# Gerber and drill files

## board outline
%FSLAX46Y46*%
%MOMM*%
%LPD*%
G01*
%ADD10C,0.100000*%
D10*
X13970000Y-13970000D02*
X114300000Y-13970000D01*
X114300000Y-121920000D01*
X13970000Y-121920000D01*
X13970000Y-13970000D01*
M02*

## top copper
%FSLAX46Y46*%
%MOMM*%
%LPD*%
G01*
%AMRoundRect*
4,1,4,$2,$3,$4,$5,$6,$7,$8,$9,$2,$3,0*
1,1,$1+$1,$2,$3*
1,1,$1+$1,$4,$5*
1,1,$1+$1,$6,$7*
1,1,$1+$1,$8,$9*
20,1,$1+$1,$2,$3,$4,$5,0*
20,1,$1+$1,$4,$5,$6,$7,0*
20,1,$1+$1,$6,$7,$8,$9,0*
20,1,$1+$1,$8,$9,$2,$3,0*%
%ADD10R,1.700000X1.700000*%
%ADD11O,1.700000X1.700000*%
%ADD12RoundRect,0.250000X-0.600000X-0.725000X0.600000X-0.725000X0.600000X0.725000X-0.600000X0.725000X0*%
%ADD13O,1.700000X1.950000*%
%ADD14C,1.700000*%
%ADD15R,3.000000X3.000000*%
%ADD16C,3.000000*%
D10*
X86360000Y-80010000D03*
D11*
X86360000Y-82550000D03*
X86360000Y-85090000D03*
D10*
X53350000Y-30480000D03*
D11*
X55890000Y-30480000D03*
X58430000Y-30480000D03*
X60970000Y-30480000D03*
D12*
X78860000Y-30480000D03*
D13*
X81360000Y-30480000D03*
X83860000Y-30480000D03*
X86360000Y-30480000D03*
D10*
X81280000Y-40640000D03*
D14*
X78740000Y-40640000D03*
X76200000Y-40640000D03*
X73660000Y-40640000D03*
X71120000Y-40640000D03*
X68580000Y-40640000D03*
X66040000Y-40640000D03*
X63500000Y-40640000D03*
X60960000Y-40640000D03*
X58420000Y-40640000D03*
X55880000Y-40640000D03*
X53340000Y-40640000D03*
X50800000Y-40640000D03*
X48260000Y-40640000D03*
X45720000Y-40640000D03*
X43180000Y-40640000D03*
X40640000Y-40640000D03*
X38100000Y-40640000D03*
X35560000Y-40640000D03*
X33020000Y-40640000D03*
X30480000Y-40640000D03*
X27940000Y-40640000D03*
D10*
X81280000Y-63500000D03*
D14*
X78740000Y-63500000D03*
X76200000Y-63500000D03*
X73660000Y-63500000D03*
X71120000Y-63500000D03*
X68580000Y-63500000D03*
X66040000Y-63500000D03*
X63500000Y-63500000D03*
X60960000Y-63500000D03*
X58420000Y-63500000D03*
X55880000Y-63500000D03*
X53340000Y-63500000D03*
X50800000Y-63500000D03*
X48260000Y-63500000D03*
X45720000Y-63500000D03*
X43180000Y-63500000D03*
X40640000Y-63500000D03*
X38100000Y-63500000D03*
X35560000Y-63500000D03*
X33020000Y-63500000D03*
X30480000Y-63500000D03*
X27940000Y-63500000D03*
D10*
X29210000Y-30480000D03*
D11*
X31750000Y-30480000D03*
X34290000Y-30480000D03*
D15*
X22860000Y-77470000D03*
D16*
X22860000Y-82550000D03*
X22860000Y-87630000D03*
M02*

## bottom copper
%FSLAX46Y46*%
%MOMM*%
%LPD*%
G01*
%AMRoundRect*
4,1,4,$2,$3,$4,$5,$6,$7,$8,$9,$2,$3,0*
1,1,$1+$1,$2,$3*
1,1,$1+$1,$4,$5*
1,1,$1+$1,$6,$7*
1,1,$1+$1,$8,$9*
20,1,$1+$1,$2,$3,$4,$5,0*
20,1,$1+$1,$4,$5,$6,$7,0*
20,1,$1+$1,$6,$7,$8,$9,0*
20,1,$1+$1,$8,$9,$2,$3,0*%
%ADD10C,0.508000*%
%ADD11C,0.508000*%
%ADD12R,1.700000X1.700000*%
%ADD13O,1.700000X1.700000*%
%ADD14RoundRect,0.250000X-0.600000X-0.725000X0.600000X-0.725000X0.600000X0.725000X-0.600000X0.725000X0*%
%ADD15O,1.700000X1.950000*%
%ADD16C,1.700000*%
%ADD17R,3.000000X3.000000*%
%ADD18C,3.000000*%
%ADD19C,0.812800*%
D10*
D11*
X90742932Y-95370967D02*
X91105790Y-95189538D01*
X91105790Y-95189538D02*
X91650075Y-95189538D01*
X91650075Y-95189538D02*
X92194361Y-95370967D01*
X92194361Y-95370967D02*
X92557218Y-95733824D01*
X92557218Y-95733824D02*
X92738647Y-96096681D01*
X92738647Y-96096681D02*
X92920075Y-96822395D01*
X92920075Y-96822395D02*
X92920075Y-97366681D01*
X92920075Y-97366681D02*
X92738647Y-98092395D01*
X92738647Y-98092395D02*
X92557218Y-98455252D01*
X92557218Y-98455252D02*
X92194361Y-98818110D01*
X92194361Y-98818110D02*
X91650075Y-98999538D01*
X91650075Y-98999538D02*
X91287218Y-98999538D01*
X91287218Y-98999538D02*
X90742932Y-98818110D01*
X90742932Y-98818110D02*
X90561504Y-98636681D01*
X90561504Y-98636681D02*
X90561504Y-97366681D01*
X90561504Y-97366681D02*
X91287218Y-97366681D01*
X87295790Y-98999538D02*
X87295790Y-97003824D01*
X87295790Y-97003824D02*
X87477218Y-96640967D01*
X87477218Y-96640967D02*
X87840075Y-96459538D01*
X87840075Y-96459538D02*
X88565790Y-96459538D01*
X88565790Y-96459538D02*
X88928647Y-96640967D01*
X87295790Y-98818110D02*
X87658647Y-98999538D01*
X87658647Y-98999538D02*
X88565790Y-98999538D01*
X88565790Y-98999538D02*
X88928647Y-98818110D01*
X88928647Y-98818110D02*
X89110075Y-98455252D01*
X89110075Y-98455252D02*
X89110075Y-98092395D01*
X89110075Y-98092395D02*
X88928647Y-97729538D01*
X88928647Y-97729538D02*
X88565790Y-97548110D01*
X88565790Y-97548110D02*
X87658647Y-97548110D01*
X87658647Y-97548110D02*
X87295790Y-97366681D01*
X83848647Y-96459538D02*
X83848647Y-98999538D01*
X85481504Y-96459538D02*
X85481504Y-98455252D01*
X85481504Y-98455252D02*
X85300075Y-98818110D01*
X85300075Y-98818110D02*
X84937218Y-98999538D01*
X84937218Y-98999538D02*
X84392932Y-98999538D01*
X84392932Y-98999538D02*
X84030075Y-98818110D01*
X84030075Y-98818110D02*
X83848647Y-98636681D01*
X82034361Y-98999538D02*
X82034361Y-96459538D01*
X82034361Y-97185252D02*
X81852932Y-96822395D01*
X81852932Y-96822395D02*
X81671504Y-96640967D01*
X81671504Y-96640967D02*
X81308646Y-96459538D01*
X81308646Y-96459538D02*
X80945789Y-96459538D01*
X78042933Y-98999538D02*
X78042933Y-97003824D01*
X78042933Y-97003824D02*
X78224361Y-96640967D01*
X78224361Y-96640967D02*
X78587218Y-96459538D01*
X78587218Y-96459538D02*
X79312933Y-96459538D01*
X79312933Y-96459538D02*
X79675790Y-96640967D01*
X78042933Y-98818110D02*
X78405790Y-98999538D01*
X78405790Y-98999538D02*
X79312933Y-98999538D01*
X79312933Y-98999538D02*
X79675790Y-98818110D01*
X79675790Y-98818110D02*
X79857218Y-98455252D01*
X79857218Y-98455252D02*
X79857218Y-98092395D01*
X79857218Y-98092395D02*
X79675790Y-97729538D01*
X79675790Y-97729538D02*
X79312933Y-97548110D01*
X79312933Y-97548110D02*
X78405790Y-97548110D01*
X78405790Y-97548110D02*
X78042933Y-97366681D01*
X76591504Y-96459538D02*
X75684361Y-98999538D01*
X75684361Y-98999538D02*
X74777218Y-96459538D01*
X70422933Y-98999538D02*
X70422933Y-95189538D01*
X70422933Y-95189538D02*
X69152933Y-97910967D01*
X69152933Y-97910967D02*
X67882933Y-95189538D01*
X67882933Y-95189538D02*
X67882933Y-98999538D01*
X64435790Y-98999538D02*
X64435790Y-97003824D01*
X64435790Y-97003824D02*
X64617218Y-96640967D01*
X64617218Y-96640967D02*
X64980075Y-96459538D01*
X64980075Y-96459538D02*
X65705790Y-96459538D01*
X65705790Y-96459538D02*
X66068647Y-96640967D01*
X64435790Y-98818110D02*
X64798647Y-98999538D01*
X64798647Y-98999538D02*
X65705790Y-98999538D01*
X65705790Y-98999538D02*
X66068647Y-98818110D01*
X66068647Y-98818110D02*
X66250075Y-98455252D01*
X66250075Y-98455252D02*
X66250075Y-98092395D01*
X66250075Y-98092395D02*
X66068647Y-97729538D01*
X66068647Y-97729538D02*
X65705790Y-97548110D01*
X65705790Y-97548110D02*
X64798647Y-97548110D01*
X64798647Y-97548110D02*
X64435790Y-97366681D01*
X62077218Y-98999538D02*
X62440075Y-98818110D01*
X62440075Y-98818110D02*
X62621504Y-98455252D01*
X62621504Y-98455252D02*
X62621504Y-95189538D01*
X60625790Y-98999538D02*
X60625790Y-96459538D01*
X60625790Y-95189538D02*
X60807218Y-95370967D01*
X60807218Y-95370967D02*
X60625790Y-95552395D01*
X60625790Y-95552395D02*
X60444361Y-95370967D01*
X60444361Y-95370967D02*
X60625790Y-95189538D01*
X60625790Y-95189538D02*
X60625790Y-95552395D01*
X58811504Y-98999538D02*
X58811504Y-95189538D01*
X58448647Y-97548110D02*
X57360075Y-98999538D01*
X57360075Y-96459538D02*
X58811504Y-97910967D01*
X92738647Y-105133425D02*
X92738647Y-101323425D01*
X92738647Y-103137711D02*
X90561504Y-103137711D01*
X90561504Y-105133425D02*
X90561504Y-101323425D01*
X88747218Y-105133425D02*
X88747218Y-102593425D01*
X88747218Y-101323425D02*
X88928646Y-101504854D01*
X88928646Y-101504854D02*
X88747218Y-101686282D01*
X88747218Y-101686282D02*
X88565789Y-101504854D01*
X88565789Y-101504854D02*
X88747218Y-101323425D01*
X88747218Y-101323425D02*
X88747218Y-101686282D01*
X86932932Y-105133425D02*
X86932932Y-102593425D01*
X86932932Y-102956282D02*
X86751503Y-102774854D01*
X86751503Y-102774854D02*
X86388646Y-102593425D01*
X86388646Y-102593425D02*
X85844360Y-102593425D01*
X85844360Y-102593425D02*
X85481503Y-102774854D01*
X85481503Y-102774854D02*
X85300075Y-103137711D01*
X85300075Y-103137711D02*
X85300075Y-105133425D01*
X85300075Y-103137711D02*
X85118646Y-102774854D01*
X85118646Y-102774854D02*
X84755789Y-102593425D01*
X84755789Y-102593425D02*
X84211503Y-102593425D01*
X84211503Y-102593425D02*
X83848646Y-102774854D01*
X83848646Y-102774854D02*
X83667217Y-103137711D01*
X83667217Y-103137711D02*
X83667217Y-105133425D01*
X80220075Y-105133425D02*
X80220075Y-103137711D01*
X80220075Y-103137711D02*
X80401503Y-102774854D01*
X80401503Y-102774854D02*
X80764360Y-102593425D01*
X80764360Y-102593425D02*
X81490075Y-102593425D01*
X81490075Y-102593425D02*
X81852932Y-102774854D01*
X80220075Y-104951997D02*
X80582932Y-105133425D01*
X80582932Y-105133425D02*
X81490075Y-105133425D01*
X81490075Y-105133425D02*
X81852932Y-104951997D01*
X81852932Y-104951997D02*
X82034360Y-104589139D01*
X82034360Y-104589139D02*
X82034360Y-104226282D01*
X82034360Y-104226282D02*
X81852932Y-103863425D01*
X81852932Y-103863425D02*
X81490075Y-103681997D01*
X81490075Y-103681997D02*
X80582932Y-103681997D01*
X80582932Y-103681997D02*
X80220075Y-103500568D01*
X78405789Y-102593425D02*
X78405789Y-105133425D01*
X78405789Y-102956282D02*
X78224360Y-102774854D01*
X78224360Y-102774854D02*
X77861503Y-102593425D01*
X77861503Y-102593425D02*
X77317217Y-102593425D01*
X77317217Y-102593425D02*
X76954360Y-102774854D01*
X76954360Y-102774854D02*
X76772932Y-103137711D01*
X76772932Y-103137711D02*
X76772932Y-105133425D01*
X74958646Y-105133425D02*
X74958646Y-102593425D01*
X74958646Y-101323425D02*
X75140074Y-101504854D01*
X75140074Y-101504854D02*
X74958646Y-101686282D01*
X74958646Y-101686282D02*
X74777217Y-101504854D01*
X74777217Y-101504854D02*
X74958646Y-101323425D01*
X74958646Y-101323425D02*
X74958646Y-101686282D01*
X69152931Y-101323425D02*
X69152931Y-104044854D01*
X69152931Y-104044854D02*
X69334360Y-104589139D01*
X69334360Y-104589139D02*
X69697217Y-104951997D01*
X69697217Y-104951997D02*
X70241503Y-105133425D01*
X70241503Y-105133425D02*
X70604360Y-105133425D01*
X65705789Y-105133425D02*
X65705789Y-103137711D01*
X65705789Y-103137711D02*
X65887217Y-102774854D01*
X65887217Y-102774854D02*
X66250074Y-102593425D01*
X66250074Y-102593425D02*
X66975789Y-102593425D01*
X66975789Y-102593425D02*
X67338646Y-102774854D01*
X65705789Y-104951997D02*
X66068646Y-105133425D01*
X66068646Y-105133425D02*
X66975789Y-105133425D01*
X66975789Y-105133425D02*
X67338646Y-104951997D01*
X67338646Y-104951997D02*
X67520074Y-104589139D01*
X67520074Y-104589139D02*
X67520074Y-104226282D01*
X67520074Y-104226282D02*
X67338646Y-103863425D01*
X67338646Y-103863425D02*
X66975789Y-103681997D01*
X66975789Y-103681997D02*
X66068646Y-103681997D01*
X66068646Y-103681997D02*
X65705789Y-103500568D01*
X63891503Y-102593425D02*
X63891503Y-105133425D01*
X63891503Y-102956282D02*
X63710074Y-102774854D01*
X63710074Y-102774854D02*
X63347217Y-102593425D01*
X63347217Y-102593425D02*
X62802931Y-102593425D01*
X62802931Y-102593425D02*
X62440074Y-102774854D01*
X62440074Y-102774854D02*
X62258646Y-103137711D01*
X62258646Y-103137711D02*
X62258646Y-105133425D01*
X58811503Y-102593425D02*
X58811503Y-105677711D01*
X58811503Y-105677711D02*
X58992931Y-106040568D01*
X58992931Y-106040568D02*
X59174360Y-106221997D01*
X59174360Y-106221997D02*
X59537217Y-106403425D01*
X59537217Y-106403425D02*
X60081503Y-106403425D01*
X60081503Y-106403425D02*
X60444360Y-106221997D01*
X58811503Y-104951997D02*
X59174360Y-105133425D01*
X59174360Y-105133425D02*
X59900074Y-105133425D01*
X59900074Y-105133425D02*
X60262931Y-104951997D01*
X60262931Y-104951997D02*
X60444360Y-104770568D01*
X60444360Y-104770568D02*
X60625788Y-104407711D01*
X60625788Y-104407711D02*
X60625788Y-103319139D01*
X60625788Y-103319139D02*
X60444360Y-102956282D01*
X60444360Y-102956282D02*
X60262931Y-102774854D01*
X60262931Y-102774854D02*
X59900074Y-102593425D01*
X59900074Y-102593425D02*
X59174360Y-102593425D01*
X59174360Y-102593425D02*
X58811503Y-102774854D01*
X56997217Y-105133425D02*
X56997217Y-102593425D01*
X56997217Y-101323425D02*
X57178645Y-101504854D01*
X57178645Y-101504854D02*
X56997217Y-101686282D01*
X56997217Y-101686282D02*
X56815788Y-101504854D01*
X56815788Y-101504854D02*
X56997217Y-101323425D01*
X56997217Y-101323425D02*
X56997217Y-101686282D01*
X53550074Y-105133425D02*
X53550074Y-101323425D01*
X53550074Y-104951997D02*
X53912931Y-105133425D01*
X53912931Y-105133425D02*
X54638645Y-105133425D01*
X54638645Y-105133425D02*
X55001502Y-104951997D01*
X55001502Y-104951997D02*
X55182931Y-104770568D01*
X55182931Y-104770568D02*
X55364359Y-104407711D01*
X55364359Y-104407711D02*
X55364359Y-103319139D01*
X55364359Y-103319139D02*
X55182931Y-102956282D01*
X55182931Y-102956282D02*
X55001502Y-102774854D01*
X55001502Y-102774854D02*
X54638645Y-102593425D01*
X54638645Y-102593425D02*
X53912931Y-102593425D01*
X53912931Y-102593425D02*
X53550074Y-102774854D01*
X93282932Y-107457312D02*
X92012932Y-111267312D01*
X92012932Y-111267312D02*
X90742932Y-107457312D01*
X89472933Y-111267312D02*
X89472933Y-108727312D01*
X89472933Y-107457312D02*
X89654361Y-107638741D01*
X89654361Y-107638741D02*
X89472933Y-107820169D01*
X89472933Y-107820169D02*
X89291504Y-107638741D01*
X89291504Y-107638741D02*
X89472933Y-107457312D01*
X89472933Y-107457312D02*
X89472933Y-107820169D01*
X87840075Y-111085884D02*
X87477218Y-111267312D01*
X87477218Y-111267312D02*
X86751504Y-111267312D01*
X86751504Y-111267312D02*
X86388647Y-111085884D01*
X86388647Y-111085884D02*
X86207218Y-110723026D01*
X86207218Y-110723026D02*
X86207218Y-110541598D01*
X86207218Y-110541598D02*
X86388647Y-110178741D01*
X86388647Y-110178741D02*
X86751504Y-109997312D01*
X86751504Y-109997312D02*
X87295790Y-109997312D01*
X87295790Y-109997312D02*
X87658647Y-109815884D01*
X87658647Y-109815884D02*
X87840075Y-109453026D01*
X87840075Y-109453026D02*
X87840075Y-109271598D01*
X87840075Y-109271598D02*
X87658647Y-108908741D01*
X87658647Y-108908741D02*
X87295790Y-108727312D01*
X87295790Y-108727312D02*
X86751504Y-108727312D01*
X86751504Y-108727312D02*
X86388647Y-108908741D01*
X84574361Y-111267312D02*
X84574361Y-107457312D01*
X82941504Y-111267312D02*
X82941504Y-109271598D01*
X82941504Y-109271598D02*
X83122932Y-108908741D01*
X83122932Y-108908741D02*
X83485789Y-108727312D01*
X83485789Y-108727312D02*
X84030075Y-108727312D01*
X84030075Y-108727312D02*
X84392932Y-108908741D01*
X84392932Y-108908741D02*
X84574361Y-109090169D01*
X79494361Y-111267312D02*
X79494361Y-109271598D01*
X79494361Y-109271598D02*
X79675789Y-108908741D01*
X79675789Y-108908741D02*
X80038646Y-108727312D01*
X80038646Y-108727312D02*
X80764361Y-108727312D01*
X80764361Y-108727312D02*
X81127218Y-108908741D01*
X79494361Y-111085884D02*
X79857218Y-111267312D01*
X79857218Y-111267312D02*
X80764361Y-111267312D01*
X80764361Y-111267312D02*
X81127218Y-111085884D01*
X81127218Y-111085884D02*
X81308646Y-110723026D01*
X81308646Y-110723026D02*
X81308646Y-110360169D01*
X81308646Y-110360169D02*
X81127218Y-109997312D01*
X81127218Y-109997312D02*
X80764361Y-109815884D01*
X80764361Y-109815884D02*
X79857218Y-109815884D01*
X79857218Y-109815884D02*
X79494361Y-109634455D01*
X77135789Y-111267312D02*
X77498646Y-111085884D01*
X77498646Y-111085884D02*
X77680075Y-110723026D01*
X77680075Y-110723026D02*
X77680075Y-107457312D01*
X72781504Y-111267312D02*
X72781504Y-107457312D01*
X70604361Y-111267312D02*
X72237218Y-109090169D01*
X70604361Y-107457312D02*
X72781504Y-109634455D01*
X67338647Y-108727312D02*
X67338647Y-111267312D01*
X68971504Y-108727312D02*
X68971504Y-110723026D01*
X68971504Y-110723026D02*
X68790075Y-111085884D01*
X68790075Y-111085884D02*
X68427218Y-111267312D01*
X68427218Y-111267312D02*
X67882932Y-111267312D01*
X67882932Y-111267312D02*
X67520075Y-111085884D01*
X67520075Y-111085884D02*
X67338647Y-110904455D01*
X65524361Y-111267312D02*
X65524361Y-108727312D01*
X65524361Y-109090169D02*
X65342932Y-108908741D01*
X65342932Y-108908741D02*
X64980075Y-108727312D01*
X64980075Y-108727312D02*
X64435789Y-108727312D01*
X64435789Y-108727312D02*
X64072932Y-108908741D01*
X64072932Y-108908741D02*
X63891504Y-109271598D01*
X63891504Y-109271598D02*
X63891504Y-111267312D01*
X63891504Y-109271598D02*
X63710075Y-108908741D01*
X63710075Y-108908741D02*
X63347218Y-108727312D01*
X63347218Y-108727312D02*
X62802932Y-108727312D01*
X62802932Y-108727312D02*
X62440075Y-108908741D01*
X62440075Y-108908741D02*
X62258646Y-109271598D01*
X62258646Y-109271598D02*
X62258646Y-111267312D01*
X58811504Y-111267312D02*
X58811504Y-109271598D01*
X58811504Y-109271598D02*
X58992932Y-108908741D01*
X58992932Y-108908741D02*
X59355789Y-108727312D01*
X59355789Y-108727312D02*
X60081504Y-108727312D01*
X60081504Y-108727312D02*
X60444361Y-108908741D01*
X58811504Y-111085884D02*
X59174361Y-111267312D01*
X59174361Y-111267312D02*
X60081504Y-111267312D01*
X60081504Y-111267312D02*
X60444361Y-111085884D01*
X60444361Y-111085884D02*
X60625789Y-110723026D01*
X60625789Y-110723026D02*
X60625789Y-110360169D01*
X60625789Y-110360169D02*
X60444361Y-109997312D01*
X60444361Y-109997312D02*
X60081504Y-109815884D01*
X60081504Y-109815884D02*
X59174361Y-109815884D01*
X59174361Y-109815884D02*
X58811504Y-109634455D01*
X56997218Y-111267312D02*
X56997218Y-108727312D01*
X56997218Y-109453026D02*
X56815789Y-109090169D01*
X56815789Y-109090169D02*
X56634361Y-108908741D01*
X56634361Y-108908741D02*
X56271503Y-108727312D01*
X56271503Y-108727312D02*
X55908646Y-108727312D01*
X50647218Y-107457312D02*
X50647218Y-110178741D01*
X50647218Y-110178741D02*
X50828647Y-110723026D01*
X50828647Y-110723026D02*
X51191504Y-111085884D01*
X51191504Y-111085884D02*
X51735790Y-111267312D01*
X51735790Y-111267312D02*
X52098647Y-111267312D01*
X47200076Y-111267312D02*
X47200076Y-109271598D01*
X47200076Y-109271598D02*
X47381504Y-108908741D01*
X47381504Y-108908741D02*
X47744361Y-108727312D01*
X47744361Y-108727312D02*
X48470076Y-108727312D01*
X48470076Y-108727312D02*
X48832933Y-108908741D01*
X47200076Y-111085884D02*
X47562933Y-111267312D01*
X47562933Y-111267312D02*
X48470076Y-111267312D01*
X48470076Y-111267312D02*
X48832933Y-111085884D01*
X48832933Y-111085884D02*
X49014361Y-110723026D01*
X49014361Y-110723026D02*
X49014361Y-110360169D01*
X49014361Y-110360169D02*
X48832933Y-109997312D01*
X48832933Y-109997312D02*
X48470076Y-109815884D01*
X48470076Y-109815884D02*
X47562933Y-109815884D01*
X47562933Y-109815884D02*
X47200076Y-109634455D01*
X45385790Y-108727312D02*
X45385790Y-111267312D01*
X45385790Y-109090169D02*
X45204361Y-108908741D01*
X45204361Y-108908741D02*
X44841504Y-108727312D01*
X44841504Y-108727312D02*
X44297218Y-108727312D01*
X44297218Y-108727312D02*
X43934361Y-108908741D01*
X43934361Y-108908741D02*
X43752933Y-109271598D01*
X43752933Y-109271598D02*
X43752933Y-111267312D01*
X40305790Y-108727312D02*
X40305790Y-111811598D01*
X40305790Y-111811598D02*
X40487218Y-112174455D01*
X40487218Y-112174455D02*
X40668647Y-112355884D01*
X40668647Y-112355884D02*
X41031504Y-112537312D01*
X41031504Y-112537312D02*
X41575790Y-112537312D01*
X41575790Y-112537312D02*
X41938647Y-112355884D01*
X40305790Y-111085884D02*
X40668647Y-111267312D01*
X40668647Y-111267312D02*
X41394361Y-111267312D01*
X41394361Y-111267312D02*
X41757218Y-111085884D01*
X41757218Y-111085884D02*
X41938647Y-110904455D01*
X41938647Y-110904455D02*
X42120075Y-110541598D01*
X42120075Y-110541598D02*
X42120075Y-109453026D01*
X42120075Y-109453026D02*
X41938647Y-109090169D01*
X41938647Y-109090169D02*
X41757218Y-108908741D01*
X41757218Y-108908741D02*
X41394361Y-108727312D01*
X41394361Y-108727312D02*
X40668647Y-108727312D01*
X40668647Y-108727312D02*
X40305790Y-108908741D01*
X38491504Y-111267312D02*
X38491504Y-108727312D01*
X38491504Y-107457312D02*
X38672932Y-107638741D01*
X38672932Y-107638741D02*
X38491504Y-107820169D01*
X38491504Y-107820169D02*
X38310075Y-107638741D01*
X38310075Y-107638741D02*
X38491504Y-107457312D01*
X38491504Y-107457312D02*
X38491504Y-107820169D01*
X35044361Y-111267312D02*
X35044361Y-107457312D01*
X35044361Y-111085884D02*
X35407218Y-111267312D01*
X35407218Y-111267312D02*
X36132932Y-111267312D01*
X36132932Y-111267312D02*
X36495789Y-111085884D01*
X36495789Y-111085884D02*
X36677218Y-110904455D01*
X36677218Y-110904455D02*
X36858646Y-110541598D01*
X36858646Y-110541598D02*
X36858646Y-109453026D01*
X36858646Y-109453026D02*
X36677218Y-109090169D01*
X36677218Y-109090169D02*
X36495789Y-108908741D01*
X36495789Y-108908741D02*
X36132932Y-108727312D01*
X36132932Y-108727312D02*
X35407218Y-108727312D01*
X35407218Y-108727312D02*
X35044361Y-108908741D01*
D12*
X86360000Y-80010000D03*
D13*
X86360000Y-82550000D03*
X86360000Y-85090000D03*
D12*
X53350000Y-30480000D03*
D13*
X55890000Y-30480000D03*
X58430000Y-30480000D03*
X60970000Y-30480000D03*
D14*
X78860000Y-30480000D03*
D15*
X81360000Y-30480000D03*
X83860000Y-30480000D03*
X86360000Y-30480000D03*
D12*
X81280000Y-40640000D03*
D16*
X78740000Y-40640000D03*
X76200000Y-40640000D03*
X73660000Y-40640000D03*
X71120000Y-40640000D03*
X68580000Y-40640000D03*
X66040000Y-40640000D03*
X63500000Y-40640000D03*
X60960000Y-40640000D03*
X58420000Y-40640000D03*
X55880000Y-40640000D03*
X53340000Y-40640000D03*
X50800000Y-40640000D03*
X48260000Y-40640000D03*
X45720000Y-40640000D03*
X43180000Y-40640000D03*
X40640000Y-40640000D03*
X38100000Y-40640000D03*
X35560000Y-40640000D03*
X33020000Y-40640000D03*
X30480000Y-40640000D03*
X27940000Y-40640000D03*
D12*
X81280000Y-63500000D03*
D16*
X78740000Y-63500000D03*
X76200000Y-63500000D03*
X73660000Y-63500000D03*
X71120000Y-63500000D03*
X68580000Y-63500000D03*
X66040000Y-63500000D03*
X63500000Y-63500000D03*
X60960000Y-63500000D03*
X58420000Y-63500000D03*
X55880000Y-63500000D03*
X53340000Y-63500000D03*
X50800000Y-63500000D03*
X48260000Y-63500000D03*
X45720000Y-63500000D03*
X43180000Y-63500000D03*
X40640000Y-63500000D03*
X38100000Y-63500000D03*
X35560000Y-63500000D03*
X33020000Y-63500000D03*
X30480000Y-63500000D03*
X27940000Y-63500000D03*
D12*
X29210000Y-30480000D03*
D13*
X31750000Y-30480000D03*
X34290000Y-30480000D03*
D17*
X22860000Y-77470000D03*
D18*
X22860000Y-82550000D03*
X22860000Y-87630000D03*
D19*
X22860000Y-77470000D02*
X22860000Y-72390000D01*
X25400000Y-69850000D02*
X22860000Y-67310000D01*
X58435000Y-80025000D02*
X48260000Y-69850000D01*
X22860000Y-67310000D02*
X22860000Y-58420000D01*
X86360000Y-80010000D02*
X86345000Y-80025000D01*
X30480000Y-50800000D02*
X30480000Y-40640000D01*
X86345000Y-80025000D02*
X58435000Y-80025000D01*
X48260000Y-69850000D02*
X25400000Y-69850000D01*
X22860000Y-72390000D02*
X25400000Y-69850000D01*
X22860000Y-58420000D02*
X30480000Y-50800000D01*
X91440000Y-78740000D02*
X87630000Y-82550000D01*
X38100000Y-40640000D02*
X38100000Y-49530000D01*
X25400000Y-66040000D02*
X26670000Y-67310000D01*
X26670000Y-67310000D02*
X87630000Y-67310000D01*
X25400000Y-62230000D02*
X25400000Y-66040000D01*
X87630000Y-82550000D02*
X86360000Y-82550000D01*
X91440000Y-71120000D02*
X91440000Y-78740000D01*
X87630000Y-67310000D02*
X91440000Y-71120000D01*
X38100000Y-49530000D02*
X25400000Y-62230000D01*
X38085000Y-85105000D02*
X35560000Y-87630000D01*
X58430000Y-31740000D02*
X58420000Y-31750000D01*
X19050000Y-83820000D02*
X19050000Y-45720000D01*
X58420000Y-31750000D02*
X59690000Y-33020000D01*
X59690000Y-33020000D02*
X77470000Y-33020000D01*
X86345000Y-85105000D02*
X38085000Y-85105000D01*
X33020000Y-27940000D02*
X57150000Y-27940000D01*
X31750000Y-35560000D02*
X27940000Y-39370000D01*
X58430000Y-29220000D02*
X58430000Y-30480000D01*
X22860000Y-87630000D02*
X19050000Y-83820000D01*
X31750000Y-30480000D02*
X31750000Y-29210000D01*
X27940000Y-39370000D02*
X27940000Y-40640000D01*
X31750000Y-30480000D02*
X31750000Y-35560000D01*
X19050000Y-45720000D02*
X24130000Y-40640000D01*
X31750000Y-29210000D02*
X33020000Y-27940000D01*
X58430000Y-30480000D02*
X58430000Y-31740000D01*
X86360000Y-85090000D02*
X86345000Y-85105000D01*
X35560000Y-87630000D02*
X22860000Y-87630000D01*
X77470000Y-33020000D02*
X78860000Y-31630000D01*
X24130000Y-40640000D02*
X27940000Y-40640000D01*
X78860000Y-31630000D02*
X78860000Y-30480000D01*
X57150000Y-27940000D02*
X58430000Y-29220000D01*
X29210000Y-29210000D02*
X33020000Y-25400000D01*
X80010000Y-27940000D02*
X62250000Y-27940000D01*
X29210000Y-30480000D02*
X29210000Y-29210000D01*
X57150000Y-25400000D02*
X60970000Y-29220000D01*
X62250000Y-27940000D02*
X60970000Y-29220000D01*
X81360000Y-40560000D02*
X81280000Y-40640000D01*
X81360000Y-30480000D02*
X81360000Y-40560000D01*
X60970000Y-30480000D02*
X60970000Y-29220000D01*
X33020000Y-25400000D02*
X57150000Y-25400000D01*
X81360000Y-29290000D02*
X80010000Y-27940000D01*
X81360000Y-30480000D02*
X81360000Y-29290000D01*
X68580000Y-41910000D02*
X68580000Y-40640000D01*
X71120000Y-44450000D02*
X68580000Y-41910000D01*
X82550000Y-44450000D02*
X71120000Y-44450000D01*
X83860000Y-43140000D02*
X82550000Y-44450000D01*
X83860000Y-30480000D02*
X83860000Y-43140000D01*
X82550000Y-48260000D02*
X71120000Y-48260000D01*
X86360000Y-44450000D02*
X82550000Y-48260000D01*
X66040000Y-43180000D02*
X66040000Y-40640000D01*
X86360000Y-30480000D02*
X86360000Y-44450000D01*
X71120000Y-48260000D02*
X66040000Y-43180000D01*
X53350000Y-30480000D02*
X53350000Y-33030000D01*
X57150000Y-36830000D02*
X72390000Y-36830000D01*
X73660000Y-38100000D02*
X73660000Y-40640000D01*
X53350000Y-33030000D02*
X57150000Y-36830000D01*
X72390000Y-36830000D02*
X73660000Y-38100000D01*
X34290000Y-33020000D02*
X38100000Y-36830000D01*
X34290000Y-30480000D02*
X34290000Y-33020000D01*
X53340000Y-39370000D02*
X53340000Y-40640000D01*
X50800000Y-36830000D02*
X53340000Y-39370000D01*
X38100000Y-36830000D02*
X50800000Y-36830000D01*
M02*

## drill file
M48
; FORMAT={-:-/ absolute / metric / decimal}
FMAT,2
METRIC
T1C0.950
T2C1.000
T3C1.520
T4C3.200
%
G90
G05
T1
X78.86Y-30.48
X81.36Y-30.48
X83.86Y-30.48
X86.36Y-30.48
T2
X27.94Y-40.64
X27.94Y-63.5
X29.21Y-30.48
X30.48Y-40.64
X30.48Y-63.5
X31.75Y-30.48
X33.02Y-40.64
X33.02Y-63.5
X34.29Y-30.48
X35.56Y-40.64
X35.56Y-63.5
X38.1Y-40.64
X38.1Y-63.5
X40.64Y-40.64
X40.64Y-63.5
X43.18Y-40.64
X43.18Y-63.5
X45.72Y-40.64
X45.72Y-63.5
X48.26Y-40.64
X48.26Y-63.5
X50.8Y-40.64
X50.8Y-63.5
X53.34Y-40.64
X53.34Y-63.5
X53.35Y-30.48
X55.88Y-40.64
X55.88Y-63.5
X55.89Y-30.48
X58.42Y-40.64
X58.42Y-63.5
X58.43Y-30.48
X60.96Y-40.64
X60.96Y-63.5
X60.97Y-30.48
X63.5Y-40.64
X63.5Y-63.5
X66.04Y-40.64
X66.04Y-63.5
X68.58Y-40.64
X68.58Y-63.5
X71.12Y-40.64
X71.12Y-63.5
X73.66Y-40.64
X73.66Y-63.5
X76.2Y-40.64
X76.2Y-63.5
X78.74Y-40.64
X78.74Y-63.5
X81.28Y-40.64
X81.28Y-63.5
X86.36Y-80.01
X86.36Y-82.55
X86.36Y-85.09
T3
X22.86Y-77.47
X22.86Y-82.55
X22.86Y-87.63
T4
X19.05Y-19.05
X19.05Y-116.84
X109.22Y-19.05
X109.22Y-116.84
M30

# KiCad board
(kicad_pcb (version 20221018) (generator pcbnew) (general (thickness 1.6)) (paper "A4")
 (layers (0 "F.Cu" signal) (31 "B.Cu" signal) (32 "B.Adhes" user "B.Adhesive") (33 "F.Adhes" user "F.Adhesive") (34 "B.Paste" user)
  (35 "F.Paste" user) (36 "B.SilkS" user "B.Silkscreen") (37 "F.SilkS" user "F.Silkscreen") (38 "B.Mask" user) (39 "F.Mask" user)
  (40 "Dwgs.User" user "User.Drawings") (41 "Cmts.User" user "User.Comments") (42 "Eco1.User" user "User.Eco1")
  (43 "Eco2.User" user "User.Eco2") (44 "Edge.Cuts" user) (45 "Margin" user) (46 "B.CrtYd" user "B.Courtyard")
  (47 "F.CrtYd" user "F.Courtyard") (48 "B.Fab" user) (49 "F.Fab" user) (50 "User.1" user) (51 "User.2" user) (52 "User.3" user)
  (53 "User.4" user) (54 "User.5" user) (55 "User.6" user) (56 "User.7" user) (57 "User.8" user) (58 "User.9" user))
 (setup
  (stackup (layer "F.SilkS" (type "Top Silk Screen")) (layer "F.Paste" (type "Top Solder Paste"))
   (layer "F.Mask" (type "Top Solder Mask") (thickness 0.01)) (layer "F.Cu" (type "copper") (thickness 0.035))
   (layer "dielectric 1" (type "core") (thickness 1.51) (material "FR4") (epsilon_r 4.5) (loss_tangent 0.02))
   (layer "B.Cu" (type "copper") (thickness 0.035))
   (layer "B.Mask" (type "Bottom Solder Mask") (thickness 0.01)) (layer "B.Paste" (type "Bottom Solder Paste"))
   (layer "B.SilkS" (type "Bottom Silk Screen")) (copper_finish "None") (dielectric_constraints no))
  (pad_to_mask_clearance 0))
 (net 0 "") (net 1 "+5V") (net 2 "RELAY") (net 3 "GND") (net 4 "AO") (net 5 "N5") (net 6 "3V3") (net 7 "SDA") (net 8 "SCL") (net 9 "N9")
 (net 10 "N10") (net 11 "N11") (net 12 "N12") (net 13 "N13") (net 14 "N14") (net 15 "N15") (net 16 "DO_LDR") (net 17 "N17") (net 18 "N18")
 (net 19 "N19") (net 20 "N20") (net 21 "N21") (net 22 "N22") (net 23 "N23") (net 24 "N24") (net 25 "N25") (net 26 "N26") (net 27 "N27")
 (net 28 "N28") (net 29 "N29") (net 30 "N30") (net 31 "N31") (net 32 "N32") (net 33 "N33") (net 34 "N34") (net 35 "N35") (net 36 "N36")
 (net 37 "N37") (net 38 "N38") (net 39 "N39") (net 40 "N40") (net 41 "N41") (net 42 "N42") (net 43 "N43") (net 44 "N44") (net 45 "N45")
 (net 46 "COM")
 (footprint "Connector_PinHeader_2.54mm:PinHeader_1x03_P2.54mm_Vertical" (layer "F.Cu") (at 86.36 80.01)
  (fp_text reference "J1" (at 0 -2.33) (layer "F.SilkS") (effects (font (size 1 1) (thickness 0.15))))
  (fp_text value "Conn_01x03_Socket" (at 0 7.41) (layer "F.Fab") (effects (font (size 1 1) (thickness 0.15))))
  (pad "1" thru_hole rect (at 0 0) (size 1.7 1.7) (drill 1) (layers "*.Cu" "*.Mask") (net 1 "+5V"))
  (pad "2" thru_hole oval (at 0 2.54) (size 1.7 1.7) (drill 1) (layers "*.Cu" "*.Mask") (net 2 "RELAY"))
  (pad "3" thru_hole oval (at 0 5.08) (size 1.7 1.7) (drill 1) (layers "*.Cu" "*.Mask") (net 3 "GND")))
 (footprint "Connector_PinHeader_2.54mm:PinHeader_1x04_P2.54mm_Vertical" (layer "F.Cu") (at 53.35 30.48 90)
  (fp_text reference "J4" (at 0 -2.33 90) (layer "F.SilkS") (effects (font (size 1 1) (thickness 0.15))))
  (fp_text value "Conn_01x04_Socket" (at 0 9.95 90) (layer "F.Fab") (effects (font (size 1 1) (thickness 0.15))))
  (pad "1" thru_hole rect (at 0 0 90) (size 1.7 1.7) (drill 1) (layers "*.Cu" "*.Mask") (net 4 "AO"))
  (pad "2" thru_hole oval (at 0 2.54 90) (size 1.7 1.7) (drill 1) (layers "*.Cu" "*.Mask") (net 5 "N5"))
  (pad "3" thru_hole oval (at 0 5.08 90) (size 1.7 1.7) (drill 1) (layers "*.Cu" "*.Mask") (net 3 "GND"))
  (pad "4" thru_hole oval (at 0 7.62 90) (size 1.7 1.7) (drill 1) (layers "*.Cu" "*.Mask") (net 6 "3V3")))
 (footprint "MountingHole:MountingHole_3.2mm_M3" (layer "F.Cu") (at 109.22 19.05)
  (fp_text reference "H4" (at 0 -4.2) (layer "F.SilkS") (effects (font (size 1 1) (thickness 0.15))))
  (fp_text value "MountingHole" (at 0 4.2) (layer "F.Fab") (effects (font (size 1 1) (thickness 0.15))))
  (pad "" np_thru_hole circle (at 0 0) (size 3.2 3.2) (drill 3.2) (layers "*.Cu" "*.Mask")))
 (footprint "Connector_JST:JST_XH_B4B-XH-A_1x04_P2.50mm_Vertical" (layer "F.Cu") (at 78.86 30.48)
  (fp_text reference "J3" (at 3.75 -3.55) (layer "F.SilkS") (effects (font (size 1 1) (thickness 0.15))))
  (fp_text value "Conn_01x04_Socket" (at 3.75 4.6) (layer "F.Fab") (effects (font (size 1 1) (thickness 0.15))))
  (pad "1" thru_hole roundrect (at 0 0) (size 1.7 1.95) (drill 0.95) (layers "*.Cu" "*.Mask") (roundrect_rratio 0.147059) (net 3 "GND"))
  (pad "2" thru_hole oval (at 2.5 0) (size 1.7 1.95) (drill 0.95) (layers "*.Cu" "*.Mask") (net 6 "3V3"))
  (pad "3" thru_hole oval (at 5 0) (size 1.7 1.95) (drill 0.95) (layers "*.Cu" "*.Mask") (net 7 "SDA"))
  (pad "4" thru_hole oval (at 7.5 0) (size 1.7 1.95) (drill 0.95) (layers "*.Cu" "*.Mask") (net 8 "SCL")))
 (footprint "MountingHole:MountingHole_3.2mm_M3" (layer "F.Cu") (at 19.05 19.05)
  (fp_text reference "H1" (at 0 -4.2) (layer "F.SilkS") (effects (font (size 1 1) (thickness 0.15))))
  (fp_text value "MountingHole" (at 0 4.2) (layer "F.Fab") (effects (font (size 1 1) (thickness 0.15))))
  (pad "" np_thru_hole circle (at 0 0) (size 3.2 3.2) (drill 3.2) (layers "*.Cu" "*.Mask")))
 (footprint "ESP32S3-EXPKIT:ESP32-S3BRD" (layer "F.Cu") (at 16.48 39.37 -90)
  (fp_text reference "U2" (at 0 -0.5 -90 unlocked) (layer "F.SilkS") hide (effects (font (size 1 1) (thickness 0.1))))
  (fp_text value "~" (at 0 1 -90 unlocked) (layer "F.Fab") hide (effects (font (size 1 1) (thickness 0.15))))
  (pad "1_1" thru_hole rect (at 1.27 -64.8 270) (size 1.7 1.7) (drill 1) (layers "*.Cu" "*.Mask") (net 6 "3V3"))
  (pad "1_2" thru_hole circle (at 1.27 -62.26 270) (size 1.7 1.7) (drill 1) (layers "*.Cu" "*.Mask") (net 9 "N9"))
  (pad "1_3" thru_hole circle (at 1.27 -59.72 270) (size 1.7 1.7) (drill 1) (layers "*.Cu" "*.Mask") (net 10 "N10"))
  (pad "1_4" thru_hole circle (at 1.27 -57.18 270) (size 1.7 1.7) (drill 1) (layers "*.Cu" "*.Mask") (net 4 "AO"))
  (pad "1_5" thru_hole circle (at 1.27 -54.64 270) (size 1.7 1.7) (drill 1) (layers "*.Cu" "*.Mask") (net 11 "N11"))
  (pad "1_6" thru_hole circle (at 1.27 -52.1 270) (size 1.7 1.7) (drill 1) (layers "*.Cu" "*.Mask") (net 7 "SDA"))
  (pad "1_7" thru_hole circle (at 1.27 -49.56 270) (size 1.7 1.7) (drill 1) (layers "*.Cu" "*.Mask") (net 8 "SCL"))
  (pad "1_8" thru_hole circle (at 1.27 -47.02 270) (size 1.7 1.7) (drill 1) (layers "*.Cu" "*.Mask") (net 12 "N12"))
  (pad "1_9" thru_hole circle (at 1.27 -44.48 270) (size 1.7 1.7) (drill 1) (layers "*.Cu" "*.Mask") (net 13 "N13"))
  (pad "1_10" thru_hole circle (at 1.27 -41.94 270) (size 1.7 1.7) (drill 1) (layers "*.Cu" "*.Mask") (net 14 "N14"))
  (pad "1_11" thru_hole circle (at 1.27 -39.4 270) (size 1.7 1.7) (drill 1) (layers "*.Cu" "*.Mask") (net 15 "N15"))
  (pad "1_12" thru_hole circle (at 1.27 -36.86 270) (size 1.7 1.7) (drill 1) (layers "*.Cu" "*.Mask") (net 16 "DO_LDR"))
  (pad "1_13" thru_hole circle (at 1.27 -34.32 270) (size 1.7 1.7) (drill 1) (layers "*.Cu" "*.Mask") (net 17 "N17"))
  (pad "1_14" thru_hole circle (at 1.27 -31.78 270) (size 1.7 1.7) (drill 1) (layers "*.Cu" "*.Mask") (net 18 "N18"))
  (pad "1_15" thru_hole circle (at 1.27 -29.24 270) (size 1.7 1.7) (drill 1) (layers "*.Cu" "*.Mask") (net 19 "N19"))
  (pad "1_16" thru_hole circle (at 1.27 -26.7 270) (size 1.7 1.7) (drill 1) (layers "*.Cu" "*.Mask") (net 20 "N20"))
  (pad "1_17" thru_hole circle (at 1.27 -24.16 270) (size 1.7 1.7) (drill 1) (layers "*.Cu" "*.Mask") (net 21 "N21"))
  (pad "1_18" thru_hole circle (at 1.27 -21.62 270) (size 1.7 1.7) (drill 1) (layers "*.Cu" "*.Mask") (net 2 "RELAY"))
  (pad "1_19" thru_hole circle (at 1.27 -19.08 270) (size 1.7 1.7) (drill 1) (layers "*.Cu" "*.Mask") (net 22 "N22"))
  (pad "1_20" thru_hole circle (at 1.27 -16.54 270) (size 1.7 1.7) (drill 1) (layers "*.Cu" "*.Mask") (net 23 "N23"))
  (pad "1_21" thru_hole circle (at 1.27 -14 270) (size 1.7 1.7) (drill 1) (layers "*.Cu" "*.Mask") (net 1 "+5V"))
  (pad "1_22" thru_hole circle (at 1.27 -11.46 270) (size 1.7 1.7) (drill 1) (layers "*.Cu" "*.Mask") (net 3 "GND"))
  (pad "2_1" thru_hole rect (at 24.13 -64.8 270) (size 1.7 1.7) (drill 1) (layers "*.Cu" "*.Mask") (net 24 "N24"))
  (pad "2_2" thru_hole circle (at 24.13 -62.26 270) (size 1.7 1.7) (drill 1) (layers "*.Cu" "*.Mask") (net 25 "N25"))
  (pad "2_3" thru_hole circle (at 24.13 -59.72 270) (size 1.7 1.7) (drill 1) (layers "*.Cu" "*.Mask") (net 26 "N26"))
  (pad "2_4" thru_hole circle (at 24.13 -57.18 270) (size 1.7 1.7) (drill 1) (layers "*.Cu" "*.Mask") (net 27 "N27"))
  (pad "2_5" thru_hole circle (at 24.13 -54.64 270) (size 1.7 1.7) (drill 1) (layers "*.Cu" "*.Mask") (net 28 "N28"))
  (pad "2_6" thru_hole circle (at 24.13 -52.1 270) (size 1.7 1.7) (drill 1) (layers "*.Cu" "*.Mask") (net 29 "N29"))
  (pad "2_7" thru_hole circle (at 24.13 -49.56 270) (size 1.7 1.7) (drill 1) (layers "*.Cu" "*.Mask") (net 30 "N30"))
  (pad "2_8" thru_hole circle (at 24.13 -47.02 270) (size 1.7 1.7) (drill 1) (layers "*.Cu" "*.Mask") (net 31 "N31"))
  (pad "2_9" thru_hole circle (at 24.13 -44.48 270) (size 1.7 1.7) (drill 1) (layers "*.Cu" "*.Mask") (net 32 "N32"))
  (pad "2_10" thru_hole circle (at 24.13 -41.94 270) (size 1.7 1.7) (drill 1) (layers "*.Cu" "*.Mask") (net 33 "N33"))
  (pad "2_11" thru_hole circle (at 24.13 -39.4 270) (size 1.7 1.7) (drill 1) (layers "*.Cu" "*.Mask") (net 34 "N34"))
  (pad "2_12" thru_hole circle (at 24.13 -36.86 270) (size 1.7 1.7) (drill 1) (layers "*.Cu" "*.Mask") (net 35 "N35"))
  (pad "2_13" thru_hole circle (at 24.13 -34.32 270) (size 1.7 1.7) (drill 1) (layers "*.Cu" "*.Mask") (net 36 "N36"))
  (pad "2_14" thru_hole circle (at 24.13 -31.78 270) (size 1.7 1.7) (drill 1) (layers "*.Cu" "*.Mask") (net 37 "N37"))
  (pad "2_15" thru_hole circle (at 24.13 -29.24 270) (size 1.7 1.7) (drill 1) (layers "*.Cu" "*.Mask") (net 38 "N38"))
  (pad "2_16" thru_hole circle (at 24.13 -26.7 270) (size 1.7 1.7) (drill 1) (layers "*.Cu" "*.Mask") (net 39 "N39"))
  (pad "2_17" thru_hole circle (at 24.13 -24.16 270) (size 1.7 1.7) (drill 1) (layers "*.Cu" "*.Mask") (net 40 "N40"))
  (pad "2_18" thru_hole circle (at 24.13 -21.62 270) (size 1.7 1.7) (drill 1) (layers "*.Cu" "*.Mask") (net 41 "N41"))
  (pad "2_19" thru_hole circle (at 24.13 -19.08 270) (size 1.7 1.7) (drill 1) (layers "*.Cu" "*.Mask") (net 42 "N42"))
  (pad "2_20" thru_hole circle (at 24.13 -16.54 270) (size 1.7 1.7) (drill 1) (layers "*.Cu" "*.Mask") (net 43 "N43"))
  (pad "2_21" thru_hole circle (at 24.13 -14 270) (size 1.7 1.7) (drill 1) (layers "*.Cu" "*.Mask") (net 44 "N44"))
  (pad "2_22" thru_hole circle (at 24.13 -11.46 270) (size 1.7 1.7) (drill 1) (layers "*.Cu" "*.Mask") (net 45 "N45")))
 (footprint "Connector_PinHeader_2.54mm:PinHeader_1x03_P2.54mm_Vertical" (layer "F.Cu") (at 29.21 30.48 90)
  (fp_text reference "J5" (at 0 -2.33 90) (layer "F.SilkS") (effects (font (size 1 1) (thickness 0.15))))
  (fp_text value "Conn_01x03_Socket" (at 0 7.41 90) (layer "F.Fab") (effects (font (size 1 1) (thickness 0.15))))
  (pad "1" thru_hole rect (at 0 0 90) (size 1.7 1.7) (drill 1) (layers "*.Cu" "*.Mask") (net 6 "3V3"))
  (pad "2" thru_hole oval (at 0 2.54 90) (size 1.7 1.7) (drill 1) (layers "*.Cu" "*.Mask") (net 3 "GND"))
  (pad "3" thru_hole oval (at 0 5.08 90) (size 1.7 1.7) (drill 1) (layers "*.Cu" "*.Mask") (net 16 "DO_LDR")))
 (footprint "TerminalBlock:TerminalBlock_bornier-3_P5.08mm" (layer "F.Cu") (at 22.86 77.47 -90)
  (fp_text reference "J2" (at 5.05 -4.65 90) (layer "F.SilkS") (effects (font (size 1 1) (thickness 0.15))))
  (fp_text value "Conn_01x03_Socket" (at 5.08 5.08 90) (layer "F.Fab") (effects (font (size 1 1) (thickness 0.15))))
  (pad "1" thru_hole rect (at 0 0 270) (size 3 3) (drill 1.52) (layers "*.Cu" "*.Mask") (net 1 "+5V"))
  (pad "2" thru_hole circle (at 5.08 0 270) (size 3 3) (drill 1.52) (layers "*.Cu" "*.Mask") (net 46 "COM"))
  (pad "3" thru_hole circle (at 10.16 0 270) (size 3 3) (drill 1.52) (layers "*.Cu" "*.Mask") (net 3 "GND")))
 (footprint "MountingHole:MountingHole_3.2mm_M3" (layer "F.Cu") (at 19.05 116.84)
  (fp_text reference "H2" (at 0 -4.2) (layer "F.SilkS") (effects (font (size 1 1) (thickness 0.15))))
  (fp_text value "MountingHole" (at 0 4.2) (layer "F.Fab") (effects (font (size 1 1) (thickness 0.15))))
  (pad "" np_thru_hole circle (at 0 0) (size 3.2 3.2) (drill 3.2) (layers "*.Cu" "*.Mask")))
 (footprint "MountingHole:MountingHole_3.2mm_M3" (layer "F.Cu") (at 109.22 116.84)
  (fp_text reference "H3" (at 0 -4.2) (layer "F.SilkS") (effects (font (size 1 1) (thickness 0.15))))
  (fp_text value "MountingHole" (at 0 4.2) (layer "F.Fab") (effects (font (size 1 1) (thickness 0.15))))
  (pad "" np_thru_hole circle (at 0 0) (size 3.2 3.2) (drill 3.2) (layers "*.Cu" "*.Mask")))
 (gr_rect (start 13.97 13.97) (end 114.3 121.92) (stroke (width 0.1) (type default)) (fill none) (layer "Edge.Cuts"))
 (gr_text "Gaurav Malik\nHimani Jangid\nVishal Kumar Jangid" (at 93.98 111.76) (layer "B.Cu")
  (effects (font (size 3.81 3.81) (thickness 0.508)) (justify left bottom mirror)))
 (segment (start 22.86 77.47) (end 22.86 72.39) (width 0.8128) (layer "B.Cu") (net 1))
 (segment (start 25.4 69.85) (end 22.86 67.31) (width 0.8128) (layer "B.Cu") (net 1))
 (segment (start 58.435 80.025) (end 48.26 69.85) (width 0.8128) (layer "B.Cu") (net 1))
 (segment (start 22.86 67.31) (end 22.86 58.42) (width 0.8128) (layer "B.Cu") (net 1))
 (segment (start 86.36 80.01) (end 86.345 80.025) (width 0.8128) (layer "B.Cu") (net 1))
 (segment (start 30.48 50.8) (end 30.48 40.64) (width 0.8128) (layer "B.Cu") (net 1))
 (segment (start 86.345 80.025) (end 58.435 80.025) (width 0.8128) (layer "B.Cu") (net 1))
 (segment (start 48.26 69.85) (end 25.4 69.85) (width 0.8128) (layer "B.Cu") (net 1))
 (segment (start 22.86 72.39) (end 25.4 69.85) (width 0.8128) (layer "B.Cu") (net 1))
 (segment (start 22.86 58.42) (end 30.48 50.8) (width 0.8128) (layer "B.Cu") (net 1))
 (segment (start 91.44 78.74) (end 87.63 82.55) (width 0.8128) (layer "B.Cu") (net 2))
 (segment (start 38.1 40.64) (end 38.1 49.53) (width 0.8128) (layer "B.Cu") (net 2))
 (segment (start 25.4 66.04) (end 26.67 67.31) (width 0.8128) (layer "B.Cu") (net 2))
 (segment (start 26.67 67.31) (end 87.63 67.31) (width 0.8128) (layer "B.Cu") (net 2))
 (segment (start 25.4 62.23) (end 25.4 66.04) (width 0.8128) (layer "B.Cu") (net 2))
 (segment (start 87.63 82.55) (end 86.36 82.55) (width 0.8128) (layer "B.Cu") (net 2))
 (segment (start 91.44 71.12) (end 91.44 78.74) (width 0.8128) (layer "B.Cu") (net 2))
 (segment (start 87.63 67.31) (end 91.44 71.12) (width 0.8128) (layer "B.Cu") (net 2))
 (segment (start 38.1 49.53) (end 25.4 62.23) (width 0.8128) (layer "B.Cu") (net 2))
 (segment (start 38.085 85.105) (end 35.56 87.63) (width 0.8128) (layer "B.Cu") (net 3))
 (segment (start 58.43 31.74) (end 58.42 31.75) (width 0.8128) (layer "B.Cu") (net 3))
 (segment (start 19.05 83.82) (end 19.05 45.72) (width 0.8128) (layer "B.Cu") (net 3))
 (segment (start 58.42 31.75) (end 59.69 33.02) (width 0.8128) (layer "B.Cu") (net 3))
 (segment (start 59.69 33.02) (end 77.47 33.02) (width 0.8128) (layer "B.Cu") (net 3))
 (segment (start 86.345 85.105) (end 38.085 85.105) (width 0.8128) (layer "B.Cu") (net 3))
 (segment (start 33.02 27.94) (end 57.15 27.94) (width 0.8128) (layer "B.Cu") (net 3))
 (segment (start 31.75 35.56) (end 27.94 39.37) (width 0.8128) (layer "B.Cu") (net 3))
 (segment (start 58.43 29.22) (end 58.43 30.48) (width 0.8128) (layer "B.Cu") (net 3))
 (segment (start 22.86 87.63) (end 19.05 83.82) (width 0.8128) (layer "B.Cu") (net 3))
 (segment (start 31.75 30.48) (end 31.75 29.21) (width 0.8128) (layer "B.Cu") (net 3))
 (segment (start 27.94 39.37) (end 27.94 40.64) (width 0.8128) (layer "B.Cu") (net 3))
 (segment (start 31.75 30.48) (end 31.75 35.56) (width 0.8128) (layer "B.Cu") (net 3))
 (segment (start 19.05 45.72) (end 24.13 40.64) (width 0.8128) (layer "B.Cu") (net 3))
 (segment (start 31.75 29.21) (end 33.02 27.94) (width 0.8128) (layer "B.Cu") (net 3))
 (segment (start 58.43 30.48) (end 58.43 31.74) (width 0.8128) (layer "B.Cu") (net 3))
 (segment (start 86.36 85.09) (end 86.345 85.105) (width 0.8128) (layer "B.Cu") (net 3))
 (segment (start 35.56 87.63) (end 22.86 87.63) (width 0.8128) (layer "B.Cu") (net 3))
 (segment (start 77.47 33.02) (end 78.86 31.63) (width 0.8128) (layer "B.Cu") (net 3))
 (segment (start 24.13 40.64) (end 27.94 40.64) (width 0.8128) (layer "B.Cu") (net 3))
 (segment (start 78.86 31.63) (end 78.86 30.48) (width 0.8128) (layer "B.Cu") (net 3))
 (segment (start 57.15 27.94) (end 58.43 29.22) (width 0.8128) (layer "B.Cu") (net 3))
 (segment (start 29.21 29.21) (end 33.02 25.4) (width 0.8128) (layer "B.Cu") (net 6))
 (segment (start 80.01 27.94) (end 62.25 27.94) (width 0.8128) (layer "B.Cu") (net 6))
 (segment (start 29.21 30.48) (end 29.21 29.21) (width 0.8128) (layer "B.Cu") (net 6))
 (segment (start 57.15 25.4) (end 60.97 29.22) (width 0.8128) (layer "B.Cu") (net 6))
 (segment (start 62.25 27.94) (end 60.97 29.22) (width 0.8128) (layer "B.Cu") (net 6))
 (segment (start 81.36 40.56) (end 81.28 40.64) (width 0.8128) (layer "B.Cu") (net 6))
 (segment (start 81.36 30.48) (end 81.36 40.56) (width 0.8128) (layer "B.Cu") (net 6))
 (segment (start 60.97 30.48) (end 60.97 29.22) (width 0.8128) (layer "B.Cu") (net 6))
 (segment (start 33.02 25.4) (end 57.15 25.4) (width 0.8128) (layer "B.Cu") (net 6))
 (segment (start 81.36 29.29) (end 80.01 27.94) (width 0.8128) (layer "B.Cu") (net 6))
 (segment (start 81.36 30.48) (end 81.36 29.29) (width 0.8128) (layer "B.Cu") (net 6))
 (segment (start 68.58 41.91) (end 68.58 40.64) (width 0.8128) (layer "B.Cu") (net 7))
 (segment (start 71.12 44.45) (end 68.58 41.91) (width 0.8128) (layer "B.Cu") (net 7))
 (segment (start 82.55 44.45) (end 71.12 44.45) (width 0.8128) (layer "B.Cu") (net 7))
 (segment (start 83.86 43.14) (end 82.55 44.45) (width 0.8128) (layer "B.Cu") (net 7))
 (segment (start 83.86 30.48) (end 83.86 43.14) (width 0.8128) (layer "B.Cu") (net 7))
 (segment (start 82.55 48.26) (end 71.12 48.26) (width 0.8128) (layer "B.Cu") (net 8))
 (segment (start 86.36 44.45) (end 82.55 48.26) (width 0.8128) (layer "B.Cu") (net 8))
 (segment (start 66.04 43.18) (end 66.04 40.64) (width 0.8128) (layer "B.Cu") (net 8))
 (segment (start 86.36 30.48) (end 86.36 44.45) (width 0.8128) (layer "B.Cu") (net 8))
 (segment (start 71.12 48.26) (end 66.04 43.18) (width 0.8128) (layer "B.Cu") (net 8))
 (segment (start 53.35 30.48) (end 53.35 33.03) (width 0.8128) (layer "B.Cu") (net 4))
 (segment (start 57.15 36.83) (end 72.39 36.83) (width 0.8128) (layer "B.Cu") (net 4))
 (segment (start 73.66 38.1) (end 73.66 40.64) (width 0.8128) (layer "B.Cu") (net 4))
 (segment (start 53.35 33.03) (end 57.15 36.83) (width 0.8128) (layer "B.Cu") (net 4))
 (segment (start 72.39 36.83) (end 73.66 38.1) (width 0.8128) (layer "B.Cu") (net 4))
 (segment (start 34.29 33.02) (end 38.1 36.83) (width 0.8128) (layer "B.Cu") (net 16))
 (segment (start 34.29 30.48) (end 34.29 33.02) (width 0.8128) (layer "B.Cu") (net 16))
 (segment (start 53.34 39.37) (end 53.34 40.64) (width 0.8128) (layer "B.Cu") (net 16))
 (segment (start 50.8 36.83) (end 53.34 39.37) (width 0.8128) (layer "B.Cu") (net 16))
 (segment (start 38.1 36.83) (end 50.8 36.83) (width 0.8128) (layer "B.Cu") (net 16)))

